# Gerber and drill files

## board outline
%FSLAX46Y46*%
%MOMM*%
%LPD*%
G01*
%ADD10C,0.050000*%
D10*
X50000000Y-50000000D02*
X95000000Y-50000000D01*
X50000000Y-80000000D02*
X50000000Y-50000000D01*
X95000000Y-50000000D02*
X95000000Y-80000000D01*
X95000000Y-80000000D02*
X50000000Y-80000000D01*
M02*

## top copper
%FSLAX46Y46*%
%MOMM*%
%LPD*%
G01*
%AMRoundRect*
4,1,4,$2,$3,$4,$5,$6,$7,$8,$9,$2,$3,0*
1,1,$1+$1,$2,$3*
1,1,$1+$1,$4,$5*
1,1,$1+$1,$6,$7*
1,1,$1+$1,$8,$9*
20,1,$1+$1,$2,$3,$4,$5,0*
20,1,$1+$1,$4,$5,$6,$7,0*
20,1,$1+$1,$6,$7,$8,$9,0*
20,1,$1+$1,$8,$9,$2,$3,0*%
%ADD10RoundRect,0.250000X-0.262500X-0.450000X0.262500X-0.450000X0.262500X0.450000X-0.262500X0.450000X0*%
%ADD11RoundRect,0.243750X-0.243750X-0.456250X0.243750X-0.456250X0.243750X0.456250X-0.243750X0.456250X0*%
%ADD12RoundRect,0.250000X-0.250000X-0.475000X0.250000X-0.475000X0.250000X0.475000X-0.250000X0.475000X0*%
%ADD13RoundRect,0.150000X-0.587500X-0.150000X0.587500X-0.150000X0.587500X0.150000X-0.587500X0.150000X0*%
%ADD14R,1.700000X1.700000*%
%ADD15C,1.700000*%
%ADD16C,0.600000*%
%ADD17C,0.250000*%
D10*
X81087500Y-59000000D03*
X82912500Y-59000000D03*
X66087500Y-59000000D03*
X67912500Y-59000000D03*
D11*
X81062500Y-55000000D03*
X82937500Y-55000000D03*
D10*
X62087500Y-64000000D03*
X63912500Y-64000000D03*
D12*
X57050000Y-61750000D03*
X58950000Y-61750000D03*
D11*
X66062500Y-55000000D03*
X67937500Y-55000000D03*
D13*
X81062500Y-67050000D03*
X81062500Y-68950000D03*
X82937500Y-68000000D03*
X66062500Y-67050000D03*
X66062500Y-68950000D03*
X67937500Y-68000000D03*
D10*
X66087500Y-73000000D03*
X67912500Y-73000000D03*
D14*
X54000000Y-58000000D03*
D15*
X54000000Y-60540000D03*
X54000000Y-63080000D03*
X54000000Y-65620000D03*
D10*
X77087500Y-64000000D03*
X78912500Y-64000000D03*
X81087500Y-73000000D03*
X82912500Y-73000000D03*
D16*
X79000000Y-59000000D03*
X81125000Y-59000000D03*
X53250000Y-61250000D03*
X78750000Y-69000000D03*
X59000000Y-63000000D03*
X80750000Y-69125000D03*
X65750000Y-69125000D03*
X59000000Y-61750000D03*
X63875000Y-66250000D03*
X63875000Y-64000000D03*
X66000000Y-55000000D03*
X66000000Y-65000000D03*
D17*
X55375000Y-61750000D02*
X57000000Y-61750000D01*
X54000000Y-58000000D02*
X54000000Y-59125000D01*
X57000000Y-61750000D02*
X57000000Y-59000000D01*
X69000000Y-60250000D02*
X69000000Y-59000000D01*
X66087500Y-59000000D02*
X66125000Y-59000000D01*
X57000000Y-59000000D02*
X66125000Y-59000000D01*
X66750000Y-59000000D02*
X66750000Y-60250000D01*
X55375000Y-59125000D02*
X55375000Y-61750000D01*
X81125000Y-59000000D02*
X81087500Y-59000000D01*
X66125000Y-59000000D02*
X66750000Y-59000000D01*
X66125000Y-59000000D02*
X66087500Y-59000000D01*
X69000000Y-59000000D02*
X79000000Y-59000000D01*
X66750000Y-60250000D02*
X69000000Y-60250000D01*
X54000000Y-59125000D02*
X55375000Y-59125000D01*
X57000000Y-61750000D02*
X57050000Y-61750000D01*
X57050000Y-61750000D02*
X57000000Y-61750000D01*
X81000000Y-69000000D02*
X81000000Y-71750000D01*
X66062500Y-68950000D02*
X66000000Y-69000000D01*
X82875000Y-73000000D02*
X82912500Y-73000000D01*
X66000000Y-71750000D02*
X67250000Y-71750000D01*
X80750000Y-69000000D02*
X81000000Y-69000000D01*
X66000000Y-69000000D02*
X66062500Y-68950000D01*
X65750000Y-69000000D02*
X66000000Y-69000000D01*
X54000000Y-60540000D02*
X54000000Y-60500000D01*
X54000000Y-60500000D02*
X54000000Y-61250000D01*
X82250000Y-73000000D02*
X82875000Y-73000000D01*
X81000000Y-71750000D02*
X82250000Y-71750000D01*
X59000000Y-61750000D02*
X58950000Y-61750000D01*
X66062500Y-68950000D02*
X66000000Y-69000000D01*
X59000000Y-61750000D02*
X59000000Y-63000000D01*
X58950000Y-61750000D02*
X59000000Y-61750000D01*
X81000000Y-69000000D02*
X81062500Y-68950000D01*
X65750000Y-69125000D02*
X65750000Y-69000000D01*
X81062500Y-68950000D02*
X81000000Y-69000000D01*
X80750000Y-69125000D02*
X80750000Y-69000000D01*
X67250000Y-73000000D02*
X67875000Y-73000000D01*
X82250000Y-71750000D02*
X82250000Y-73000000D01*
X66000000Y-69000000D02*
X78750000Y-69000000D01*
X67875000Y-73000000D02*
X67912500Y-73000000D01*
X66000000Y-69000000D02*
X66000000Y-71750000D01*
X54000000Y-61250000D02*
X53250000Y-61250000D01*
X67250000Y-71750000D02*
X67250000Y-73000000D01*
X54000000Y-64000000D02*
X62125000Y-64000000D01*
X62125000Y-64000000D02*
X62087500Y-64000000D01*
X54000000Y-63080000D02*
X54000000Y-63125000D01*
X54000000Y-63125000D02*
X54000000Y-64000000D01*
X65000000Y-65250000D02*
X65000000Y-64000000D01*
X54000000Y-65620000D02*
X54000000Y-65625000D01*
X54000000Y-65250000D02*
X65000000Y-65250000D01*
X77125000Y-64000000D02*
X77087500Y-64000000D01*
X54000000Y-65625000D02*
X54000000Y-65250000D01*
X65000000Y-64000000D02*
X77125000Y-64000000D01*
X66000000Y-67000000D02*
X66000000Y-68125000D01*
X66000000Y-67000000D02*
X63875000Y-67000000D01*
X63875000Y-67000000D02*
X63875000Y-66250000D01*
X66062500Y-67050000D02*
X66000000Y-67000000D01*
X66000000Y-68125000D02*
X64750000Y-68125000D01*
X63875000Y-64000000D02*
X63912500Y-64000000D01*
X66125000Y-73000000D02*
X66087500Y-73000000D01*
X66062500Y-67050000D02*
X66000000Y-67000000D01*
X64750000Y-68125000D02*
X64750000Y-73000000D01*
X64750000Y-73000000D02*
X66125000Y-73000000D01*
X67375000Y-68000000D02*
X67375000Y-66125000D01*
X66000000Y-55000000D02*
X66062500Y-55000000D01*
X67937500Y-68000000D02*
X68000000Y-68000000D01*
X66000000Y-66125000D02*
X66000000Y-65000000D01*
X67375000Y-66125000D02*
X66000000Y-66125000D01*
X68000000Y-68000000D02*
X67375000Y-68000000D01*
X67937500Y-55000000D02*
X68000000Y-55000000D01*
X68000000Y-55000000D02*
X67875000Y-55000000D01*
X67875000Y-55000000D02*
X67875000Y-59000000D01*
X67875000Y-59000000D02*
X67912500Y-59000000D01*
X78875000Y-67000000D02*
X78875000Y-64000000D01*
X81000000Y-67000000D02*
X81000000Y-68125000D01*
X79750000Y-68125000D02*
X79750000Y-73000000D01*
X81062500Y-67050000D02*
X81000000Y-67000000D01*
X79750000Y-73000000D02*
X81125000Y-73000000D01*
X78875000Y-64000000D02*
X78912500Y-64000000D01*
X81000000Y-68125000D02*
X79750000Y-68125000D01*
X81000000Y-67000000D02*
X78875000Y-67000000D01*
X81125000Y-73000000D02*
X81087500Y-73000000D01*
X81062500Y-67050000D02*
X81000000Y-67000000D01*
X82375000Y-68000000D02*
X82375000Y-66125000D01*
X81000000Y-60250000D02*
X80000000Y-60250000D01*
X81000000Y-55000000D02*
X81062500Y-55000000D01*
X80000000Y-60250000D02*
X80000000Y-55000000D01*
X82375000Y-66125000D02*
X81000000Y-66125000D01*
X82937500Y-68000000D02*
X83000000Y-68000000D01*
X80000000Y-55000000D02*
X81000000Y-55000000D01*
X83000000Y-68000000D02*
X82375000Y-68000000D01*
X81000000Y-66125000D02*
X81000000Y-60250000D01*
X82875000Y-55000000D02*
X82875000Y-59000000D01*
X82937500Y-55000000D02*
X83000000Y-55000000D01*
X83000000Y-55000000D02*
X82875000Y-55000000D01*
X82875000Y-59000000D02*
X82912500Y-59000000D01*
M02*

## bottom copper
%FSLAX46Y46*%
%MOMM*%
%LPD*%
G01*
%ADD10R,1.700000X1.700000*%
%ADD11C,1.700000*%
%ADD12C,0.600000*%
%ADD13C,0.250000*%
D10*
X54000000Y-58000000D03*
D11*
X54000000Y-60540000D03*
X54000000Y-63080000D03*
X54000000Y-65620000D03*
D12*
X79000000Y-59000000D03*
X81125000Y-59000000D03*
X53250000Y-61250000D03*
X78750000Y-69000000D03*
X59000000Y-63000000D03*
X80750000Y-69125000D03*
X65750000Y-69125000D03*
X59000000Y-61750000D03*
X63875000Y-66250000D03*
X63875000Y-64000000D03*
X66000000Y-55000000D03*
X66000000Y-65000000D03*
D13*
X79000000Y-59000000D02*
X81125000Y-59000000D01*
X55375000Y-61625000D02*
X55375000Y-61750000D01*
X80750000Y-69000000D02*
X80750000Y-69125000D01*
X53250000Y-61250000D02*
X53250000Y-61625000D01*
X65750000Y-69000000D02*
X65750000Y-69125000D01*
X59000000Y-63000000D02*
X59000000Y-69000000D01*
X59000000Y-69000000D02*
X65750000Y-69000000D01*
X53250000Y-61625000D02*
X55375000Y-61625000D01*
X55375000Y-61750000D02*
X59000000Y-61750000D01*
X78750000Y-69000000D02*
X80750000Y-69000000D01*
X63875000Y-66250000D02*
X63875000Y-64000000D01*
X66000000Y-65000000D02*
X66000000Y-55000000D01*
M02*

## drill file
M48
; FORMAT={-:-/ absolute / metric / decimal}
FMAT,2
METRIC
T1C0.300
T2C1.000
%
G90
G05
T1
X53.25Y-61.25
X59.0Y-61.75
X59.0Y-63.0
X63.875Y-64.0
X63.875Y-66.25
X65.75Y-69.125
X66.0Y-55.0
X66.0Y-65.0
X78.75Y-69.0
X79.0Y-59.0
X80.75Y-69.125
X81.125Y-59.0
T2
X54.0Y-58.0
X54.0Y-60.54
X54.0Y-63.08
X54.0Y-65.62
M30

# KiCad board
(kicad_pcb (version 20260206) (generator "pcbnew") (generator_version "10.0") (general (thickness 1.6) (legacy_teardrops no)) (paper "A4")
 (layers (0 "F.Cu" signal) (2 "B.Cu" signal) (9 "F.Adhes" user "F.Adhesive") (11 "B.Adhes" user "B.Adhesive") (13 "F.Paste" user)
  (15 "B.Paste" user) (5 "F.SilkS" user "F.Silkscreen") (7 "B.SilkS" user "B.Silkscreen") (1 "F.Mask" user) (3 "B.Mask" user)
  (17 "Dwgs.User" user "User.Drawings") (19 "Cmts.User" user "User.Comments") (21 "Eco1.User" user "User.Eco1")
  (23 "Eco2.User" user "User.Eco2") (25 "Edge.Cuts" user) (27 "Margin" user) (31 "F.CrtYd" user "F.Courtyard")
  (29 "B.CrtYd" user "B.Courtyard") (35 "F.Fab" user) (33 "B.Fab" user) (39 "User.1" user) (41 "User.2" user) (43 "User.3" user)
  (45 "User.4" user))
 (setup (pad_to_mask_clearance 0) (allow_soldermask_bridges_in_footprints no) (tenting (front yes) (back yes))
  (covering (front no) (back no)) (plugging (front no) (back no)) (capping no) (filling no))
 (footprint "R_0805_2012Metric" (layer "F.Cu") (at 82 59)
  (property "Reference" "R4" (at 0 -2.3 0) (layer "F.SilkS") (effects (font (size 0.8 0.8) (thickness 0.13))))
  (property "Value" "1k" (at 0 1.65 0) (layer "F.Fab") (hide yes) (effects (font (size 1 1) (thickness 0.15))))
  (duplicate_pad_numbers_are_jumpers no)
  (pad "1" smd roundrect (at -0.9125 0) (size 1.025 1.4) (layers "F.Cu" "F.Mask" "F.Paste") (roundrect_rratio 0.243902) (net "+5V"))
  (pad "2" smd roundrect (at 0.9125 0) (size 1.025 1.4) (layers "F.Cu" "F.Mask" "F.Paste") (roundrect_rratio 0.243902) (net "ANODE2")))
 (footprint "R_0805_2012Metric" (layer "F.Cu") (at 67 59)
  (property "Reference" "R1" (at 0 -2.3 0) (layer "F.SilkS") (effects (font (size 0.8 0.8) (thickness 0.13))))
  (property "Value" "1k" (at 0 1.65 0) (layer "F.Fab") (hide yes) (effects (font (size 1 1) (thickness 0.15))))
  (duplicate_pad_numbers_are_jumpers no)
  (pad "1" smd roundrect (at -0.9125 0) (size 1.025 1.4) (layers "F.Cu" "F.Mask" "F.Paste") (roundrect_rratio 0.243902) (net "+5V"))
  (pad "2" smd roundrect (at 0.9125 0) (size 1.025 1.4) (layers "F.Cu" "F.Mask" "F.Paste") (roundrect_rratio 0.243902) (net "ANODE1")))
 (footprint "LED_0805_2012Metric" (layer "F.Cu") (at 82 55)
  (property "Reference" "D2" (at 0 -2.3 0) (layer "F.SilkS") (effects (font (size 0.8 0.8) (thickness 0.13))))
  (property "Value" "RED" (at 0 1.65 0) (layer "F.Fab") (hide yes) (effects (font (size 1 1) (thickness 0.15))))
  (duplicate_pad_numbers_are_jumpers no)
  (pad "1" smd roundrect (at -0.9375 0) (size 0.975 1.4) (layers "F.Cu" "F.Mask" "F.Paste") (roundrect_rratio 0.25) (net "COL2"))
  (pad "2" smd roundrect (at 0.9375 0) (size 0.975 1.4) (layers "F.Cu" "F.Mask" "F.Paste") (roundrect_rratio 0.25) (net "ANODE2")))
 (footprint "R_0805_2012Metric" (layer "F.Cu") (at 63 64)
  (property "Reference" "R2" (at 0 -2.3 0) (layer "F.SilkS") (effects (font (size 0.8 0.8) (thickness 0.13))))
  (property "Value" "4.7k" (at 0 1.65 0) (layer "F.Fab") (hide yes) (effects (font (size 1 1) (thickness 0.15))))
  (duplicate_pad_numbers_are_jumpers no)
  (pad "1" smd roundrect (at -0.9125 0) (size 1.025 1.4) (layers "F.Cu" "F.Mask" "F.Paste") (roundrect_rratio 0.243902) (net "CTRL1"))
  (pad "2" smd roundrect (at 0.9125 0) (size 1.025 1.4) (layers "F.Cu" "F.Mask" "F.Paste") (roundrect_rratio 0.243902) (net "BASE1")))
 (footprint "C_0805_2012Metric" (layer "F.Cu") (at 58 61.75)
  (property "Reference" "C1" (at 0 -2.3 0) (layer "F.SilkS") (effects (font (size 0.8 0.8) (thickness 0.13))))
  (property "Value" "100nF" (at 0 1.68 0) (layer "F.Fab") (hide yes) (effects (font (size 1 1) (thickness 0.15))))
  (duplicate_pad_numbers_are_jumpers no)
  (pad "1" smd roundrect (at -0.95 0) (size 1 1.45) (layers "F.Cu" "F.Mask" "F.Paste") (roundrect_rratio 0.25) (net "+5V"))
  (pad "2" smd roundrect (at 0.95 0) (size 1 1.45) (layers "F.Cu" "F.Mask" "F.Paste") (roundrect_rratio 0.25) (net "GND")))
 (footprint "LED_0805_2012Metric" (layer "F.Cu") (at 67 55)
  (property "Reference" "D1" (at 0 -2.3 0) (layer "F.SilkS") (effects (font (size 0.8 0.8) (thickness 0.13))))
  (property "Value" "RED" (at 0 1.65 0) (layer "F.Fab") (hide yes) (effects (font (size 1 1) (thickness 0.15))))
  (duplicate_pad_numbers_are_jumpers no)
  (pad "1" smd roundrect (at -0.9375 0) (size 0.975 1.4) (layers "F.Cu" "F.Mask" "F.Paste") (roundrect_rratio 0.25) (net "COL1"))
  (pad "2" smd roundrect (at 0.9375 0) (size 0.975 1.4) (layers "F.Cu" "F.Mask" "F.Paste") (roundrect_rratio 0.25) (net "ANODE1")))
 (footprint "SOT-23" (layer "F.Cu") (at 82 68)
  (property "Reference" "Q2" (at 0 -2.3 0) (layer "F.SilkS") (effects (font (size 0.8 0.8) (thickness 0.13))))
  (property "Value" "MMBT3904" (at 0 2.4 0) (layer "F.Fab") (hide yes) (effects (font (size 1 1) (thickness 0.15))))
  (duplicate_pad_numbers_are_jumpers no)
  (pad "1" smd roundrect (at -0.9375 -0.95) (size 1.475 0.6) (layers "F.Cu" "F.Mask" "F.Paste") (roundrect_rratio 0.25) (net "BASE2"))
  (pad "2" smd roundrect (at -0.9375 0.95) (size 1.475 0.6) (layers "F.Cu" "F.Mask" "F.Paste") (roundrect_rratio 0.25) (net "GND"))
  (pad "3" smd roundrect (at 0.9375 0) (size 1.475 0.6) (layers "F.Cu" "F.Mask" "F.Paste") (roundrect_rratio 0.25) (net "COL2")))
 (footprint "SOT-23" (layer "F.Cu") (at 67 68)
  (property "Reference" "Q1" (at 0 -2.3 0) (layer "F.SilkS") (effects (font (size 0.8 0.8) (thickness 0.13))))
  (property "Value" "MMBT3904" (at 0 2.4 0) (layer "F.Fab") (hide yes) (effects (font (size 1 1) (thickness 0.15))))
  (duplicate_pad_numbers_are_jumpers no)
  (pad "1" smd roundrect (at -0.9375 -0.95) (size 1.475 0.6) (layers "F.Cu" "F.Mask" "F.Paste") (roundrect_rratio 0.25) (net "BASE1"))
  (pad "2" smd roundrect (at -0.9375 0.95) (size 1.475 0.6) (layers "F.Cu" "F.Mask" "F.Paste") (roundrect_rratio 0.25) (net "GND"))
  (pad "3" smd roundrect (at 0.9375 0) (size 1.475 0.6) (layers "F.Cu" "F.Mask" "F.Paste") (roundrect_rratio 0.25) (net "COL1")))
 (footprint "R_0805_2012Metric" (layer "F.Cu") (at 67 73)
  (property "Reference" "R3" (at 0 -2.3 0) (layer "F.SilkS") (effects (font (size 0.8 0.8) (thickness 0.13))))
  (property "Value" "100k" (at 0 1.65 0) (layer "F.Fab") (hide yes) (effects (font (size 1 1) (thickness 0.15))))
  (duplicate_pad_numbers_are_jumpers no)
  (pad "1" smd roundrect (at -0.9125 0) (size 1.025 1.4) (layers "F.Cu" "F.Mask" "F.Paste") (roundrect_rratio 0.243902) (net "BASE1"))
  (pad "2" smd roundrect (at 0.9125 0) (size 1.025 1.4) (layers "F.Cu" "F.Mask" "F.Paste") (roundrect_rratio 0.243902) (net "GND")))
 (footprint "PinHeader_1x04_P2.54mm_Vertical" (layer "F.Cu") (at 54 58)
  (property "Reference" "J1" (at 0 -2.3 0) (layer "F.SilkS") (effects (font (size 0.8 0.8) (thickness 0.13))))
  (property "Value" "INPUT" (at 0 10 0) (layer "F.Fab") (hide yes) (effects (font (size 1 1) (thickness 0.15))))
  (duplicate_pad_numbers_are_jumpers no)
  (pad "1" thru_hole rect (at 0 0) (size 1.7 1.7) (drill 1) (layers "*.Cu" "*.Mask") (remove_unused_layers no) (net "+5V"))
  (pad "2" thru_hole circle (at 0 2.54) (size 1.7 1.7) (drill 1) (layers "*.Cu" "*.Mask") (remove_unused_layers no) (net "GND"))
  (pad "3" thru_hole circle (at 0 5.08) (size 1.7 1.7) (drill 1) (layers "*.Cu" "*.Mask") (remove_unused_layers no) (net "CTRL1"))
  (pad "4" thru_hole circle (at 0 7.62) (size 1.7 1.7) (drill 1) (layers "*.Cu" "*.Mask") (remove_unused_layers no) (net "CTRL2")))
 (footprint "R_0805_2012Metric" (layer "F.Cu") (at 78 64)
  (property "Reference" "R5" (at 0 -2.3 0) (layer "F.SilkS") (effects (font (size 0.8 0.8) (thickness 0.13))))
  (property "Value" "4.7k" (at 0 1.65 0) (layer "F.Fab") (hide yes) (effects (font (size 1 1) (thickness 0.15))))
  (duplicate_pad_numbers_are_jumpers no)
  (pad "1" smd roundrect (at -0.9125 0) (size 1.025 1.4) (layers "F.Cu" "F.Mask" "F.Paste") (roundrect_rratio 0.243902) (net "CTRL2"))
  (pad "2" smd roundrect (at 0.9125 0) (size 1.025 1.4) (layers "F.Cu" "F.Mask" "F.Paste") (roundrect_rratio 0.243902) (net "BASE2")))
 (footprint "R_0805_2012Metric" (layer "F.Cu") (at 82 73)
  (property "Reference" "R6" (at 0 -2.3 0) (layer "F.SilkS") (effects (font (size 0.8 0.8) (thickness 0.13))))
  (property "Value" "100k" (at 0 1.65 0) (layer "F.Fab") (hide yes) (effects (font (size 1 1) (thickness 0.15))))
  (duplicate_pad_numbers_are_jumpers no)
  (pad "1" smd roundrect (at -0.9125 0) (size 1.025 1.4) (layers "F.Cu" "F.Mask" "F.Paste") (roundrect_rratio 0.243902) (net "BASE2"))
  (pad "2" smd roundrect (at 0.9125 0) (size 1.025 1.4) (layers "F.Cu" "F.Mask" "F.Paste") (roundrect_rratio 0.243902) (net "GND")))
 (gr_line (start 50 50) (end 95 50) (stroke (width 0.05) (type default)) (layer "Edge.Cuts"))
 (gr_line (start 50 80) (end 50 50) (stroke (width 0.05) (type default)) (layer "Edge.Cuts"))
 (gr_line (start 95 50) (end 95 80) (stroke (width 0.05) (type default)) (layer "Edge.Cuts"))
 (gr_line (start 95 80) (end 50 80) (stroke (width 0.05) (type default)) (layer "Edge.Cuts"))
 (segment (start 55.375 61.75) (end 57 61.75) (width 0.25) (layer "F.Cu") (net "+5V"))
 (segment (start 54 58) (end 54 59.125) (width 0.25) (layer "F.Cu") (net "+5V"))
 (segment (start 57 61.75) (end 57 59) (width 0.25) (layer "F.Cu") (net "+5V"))
 (segment (start 69 60.25) (end 69 59) (width 0.25) (layer "F.Cu") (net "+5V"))
 (segment (start 66.0875 59) (end 66.125 59) (width 0.25) (layer "F.Cu") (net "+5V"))
 (segment (start 57 59) (end 66.125 59) (width 0.25) (layer "F.Cu") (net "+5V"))
 (segment (start 66.75 59) (end 66.75 60.25) (width 0.25) (layer "F.Cu") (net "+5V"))
 (segment (start 55.375 59.125) (end 55.375 61.75) (width 0.25) (layer "F.Cu") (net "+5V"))
 (segment (start 81.125 59) (end 81.0875 59) (width 0.25) (layer "F.Cu") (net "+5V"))
 (segment (start 66.125 59) (end 66.75 59) (width 0.25) (layer "F.Cu") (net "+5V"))
 (segment (start 66.125 59) (end 66.0875 59) (width 0.25) (layer "F.Cu") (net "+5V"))
 (segment (start 69 59) (end 79 59) (width 0.25) (layer "F.Cu") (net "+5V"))
 (segment (start 66.75 60.25) (end 69 60.25) (width 0.25) (layer "F.Cu") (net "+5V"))
 (segment (start 54 59.125) (end 55.375 59.125) (width 0.25) (layer "F.Cu") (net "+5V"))
 (segment (start 57 61.75) (end 57.05 61.75) (width 0.25) (layer "F.Cu") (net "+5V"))
 (segment (start 57.05 61.75) (end 57 61.75) (width 0.25) (layer "F.Cu") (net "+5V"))
 (via (at 79 59) (size 0.6) (drill 0.3) (layers "F.Cu" "B.Cu") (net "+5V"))
 (via (at 81.125 59) (size 0.6) (drill 0.3) (layers "F.Cu" "B.Cu") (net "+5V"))
 (segment (start 79 59) (end 81.125 59) (width 0.25) (layer "B.Cu") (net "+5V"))
 (segment (start 81 69) (end 81 71.75) (width 0.25) (layer "F.Cu") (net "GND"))
 (segment (start 66.0625 68.95) (end 66 69) (width 0.25) (layer "F.Cu") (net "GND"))
 (segment (start 82.875 73) (end 82.9125 73) (width 0.25) (layer "F.Cu") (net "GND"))
 (segment (start 66 71.75) (end 67.25 71.75) (width 0.25) (layer "F.Cu") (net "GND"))
 (segment (start 80.75 69) (end 81 69) (width 0.25) (layer "F.Cu") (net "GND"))
 (segment (start 66 69) (end 66.0625 68.95) (width 0.25) (layer "F.Cu") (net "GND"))
 (segment (start 65.75 69) (end 66 69) (width 0.25) (layer "F.Cu") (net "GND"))
 (segment (start 54 60.54) (end 54 60.5) (width 0.25) (layer "F.Cu") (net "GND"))
 (segment (start 54 60.5) (end 54 61.25) (width 0.25) (layer "F.Cu") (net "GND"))
 (segment (start 82.25 73) (end 82.875 73) (width 0.25) (layer "F.Cu") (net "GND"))
 (segment (start 81 71.75) (end 82.25 71.75) (width 0.25) (layer "F.Cu") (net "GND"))
 (segment (start 59 61.75) (end 58.95 61.75) (width 0.25) (layer "F.Cu") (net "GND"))
 (segment (start 66.0625 68.95) (end 66 69) (width 0.25) (layer "F.Cu") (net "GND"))
 (segment (start 59 61.75) (end 59 63) (width 0.25) (layer "F.Cu") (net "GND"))
 (segment (start 58.95 61.75) (end 59 61.75) (width 0.25) (layer "F.Cu") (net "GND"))
 (segment (start 81 69) (end 81.0625 68.95) (width 0.25) (layer "F.Cu") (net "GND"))
 (segment (start 65.75 69.125) (end 65.75 69) (width 0.25) (layer "F.Cu") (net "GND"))
 (segment (start 81.0625 68.95) (end 81 69) (width 0.25) (layer "F.Cu") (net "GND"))
 (segment (start 80.75 69.125) (end 80.75 69) (width 0.25) (layer "F.Cu") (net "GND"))
 (segment (start 67.25 73) (end 67.875 73) (width 0.25) (layer "F.Cu") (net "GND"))
 (segment (start 82.25 71.75) (end 82.25 73) (width 0.25) (layer "F.Cu") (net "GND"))
 (segment (start 66 69) (end 78.75 69) (width 0.25) (layer "F.Cu") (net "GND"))
 (segment (start 67.875 73) (end 67.9125 73) (width 0.25) (layer "F.Cu") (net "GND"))
 (segment (start 66 69) (end 66 71.75) (width 0.25) (layer "F.Cu") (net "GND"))
 (segment (start 54 61.25) (end 53.25 61.25) (width 0.25) (layer "F.Cu") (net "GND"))
 (segment (start 67.25 71.75) (end 67.25 73) (width 0.25) (layer "F.Cu") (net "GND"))
 (via (at 53.25 61.25) (size 0.6) (drill 0.3) (layers "F.Cu" "B.Cu") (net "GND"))
 (via (at 78.75 69) (size 0.6) (drill 0.3) (layers "F.Cu" "B.Cu") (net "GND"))
 (via (at 59 63) (size 0.6) (drill 0.3) (layers "F.Cu" "B.Cu") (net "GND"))
 (via (at 80.75 69.125) (size 0.6) (drill 0.3) (layers "F.Cu" "B.Cu") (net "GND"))
 (via (at 65.75 69.125) (size 0.6) (drill 0.3) (layers "F.Cu" "B.Cu") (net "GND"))
 (via (at 59 61.75) (size 0.6) (drill 0.3) (layers "F.Cu" "B.Cu") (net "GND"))
 (segment (start 55.375 61.625) (end 55.375 61.75) (width 0.25) (layer "B.Cu") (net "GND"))
 (segment (start 80.75 69) (end 80.75 69.125) (width 0.25) (layer "B.Cu") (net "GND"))
 (segment (start 53.25 61.25) (end 53.25 61.625) (width 0.25) (layer "B.Cu") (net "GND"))
 (segment (start 65.75 69) (end 65.75 69.125) (width 0.25) (layer "B.Cu") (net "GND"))
 (segment (start 59 63) (end 59 69) (width 0.25) (layer "B.Cu") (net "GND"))
 (segment (start 59 69) (end 65.75 69) (width 0.25) (layer "B.Cu") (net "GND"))
 (segment (start 53.25 61.625) (end 55.375 61.625) (width 0.25) (layer "B.Cu") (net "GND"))
 (segment (start 55.375 61.75) (end 59 61.75) (width 0.25) (layer "B.Cu") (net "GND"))
 (segment (start 78.75 69) (end 80.75 69) (width 0.25) (layer "B.Cu") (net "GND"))
 (segment (start 54 64) (end 62.125 64) (width 0.25) (layer "F.Cu") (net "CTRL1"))
 (segment (start 62.125 64) (end 62.0875 64) (width 0.25) (layer "F.Cu") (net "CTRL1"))
 (segment (start 54 63.08) (end 54 63.125) (width 0.25) (layer "F.Cu") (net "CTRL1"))
 (segment (start 54 63.125) (end 54 64) (width 0.25) (layer "F.Cu") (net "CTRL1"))
 (segment (start 65 65.25) (end 65 64) (width 0.25) (layer "F.Cu") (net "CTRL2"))
 (segment (start 54 65.62) (end 54 65.625) (width 0.25) (layer "F.Cu") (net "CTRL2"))
 (segment (start 54 65.25) (end 65 65.25) (width 0.25) (layer "F.Cu") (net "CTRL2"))
 (segment (start 77.125 64) (end 77.0875 64) (width 0.25) (layer "F.Cu") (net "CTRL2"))
 (segment (start 54 65.625) (end 54 65.25) (width 0.25) (layer "F.Cu") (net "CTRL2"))
 (segment (start 65 64) (end 77.125 64) (width 0.25) (layer "F.Cu") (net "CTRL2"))
 (segment (start 66 67) (end 66 68.125) (width 0.25) (layer "F.Cu") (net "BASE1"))
 (segment (start 66 67) (end 63.875 67) (width 0.25) (layer "F.Cu") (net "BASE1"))
 (segment (start 63.875 67) (end 63.875 66.25) (width 0.25) (layer "F.Cu") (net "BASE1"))
 (segment (start 66.0625 67.05) (end 66 67) (width 0.25) (layer "F.Cu") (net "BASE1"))
 (segment (start 66 68.125) (end 64.75 68.125) (width 0.25) (layer "F.Cu") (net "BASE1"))
 (segment (start 63.875 64) (end 63.9125 64) (width 0.25) (layer "F.Cu") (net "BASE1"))
 (segment (start 66.125 73) (end 66.0875 73) (width 0.25) (layer "F.Cu") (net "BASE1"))
 (segment (start 66.0625 67.05) (end 66 67) (width 0.25) (layer "F.Cu") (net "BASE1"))
 (segment (start 64.75 68.125) (end 64.75 73) (width 0.25) (layer "F.Cu") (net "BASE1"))
 (segment (start 64.75 73) (end 66.125 73) (width 0.25) (layer "F.Cu") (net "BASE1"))
 (via (at 63.875 66.25) (size 0.6) (drill 0.3) (layers "F.Cu" "B.Cu") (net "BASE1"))
 (via (at 63.875 64) (size 0.6) (drill 0.3) (layers "F.Cu" "B.Cu") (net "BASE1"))
 (segment (start 63.875 66.25) (end 63.875 64) (width 0.25) (layer "B.Cu") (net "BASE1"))
 (segment (start 67.375 68) (end 67.375 66.125) (width 0.25) (layer "F.Cu") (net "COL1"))
 (segment (start 66 55) (end 66.0625 55) (width 0.25) (layer "F.Cu") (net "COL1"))
 (segment (start 67.9375 68) (end 68 68) (width 0.25) (layer "F.Cu") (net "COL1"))
 (segment (start 66 66.125) (end 66 65) (width 0.25) (layer "F.Cu") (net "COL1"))
 (segment (start 67.375 66.125) (end 66 66.125) (width 0.25) (layer "F.Cu") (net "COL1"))
 (segment (start 68 68) (end 67.375 68) (width 0.25) (layer "F.Cu") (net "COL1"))
 (via (at 66 55) (size 0.6) (drill 0.3) (layers "F.Cu" "B.Cu") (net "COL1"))
 (via (at 66 65) (size 0.6) (drill 0.3) (layers "F.Cu" "B.Cu") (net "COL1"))
 (segment (start 66 65) (end 66 55) (width 0.25) (layer "B.Cu") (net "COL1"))
 (segment (start 67.9375 55) (end 68 55) (width 0.25) (layer "F.Cu") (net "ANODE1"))
 (segment (start 68 55) (end 67.875 55) (width 0.25) (layer "F.Cu") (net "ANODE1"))
 (segment (start 67.875 55) (end 67.875 59) (width 0.25) (layer "F.Cu") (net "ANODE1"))
 (segment (start 67.875 59) (end 67.9125 59) (width 0.25) (layer "F.Cu") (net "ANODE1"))
 (segment (start 78.875 67) (end 78.875 64) (width 0.25) (layer "F.Cu") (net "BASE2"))
 (segment (start 81 67) (end 81 68.125) (width 0.25) (layer "F.Cu") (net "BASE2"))
 (segment (start 79.75 68.125) (end 79.75 73) (width 0.25) (layer "F.Cu") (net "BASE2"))
 (segment (start 81.0625 67.05) (end 81 67) (width 0.25) (layer "F.Cu") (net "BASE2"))
 (segment (start 79.75 73) (end 81.125 73) (width 0.25) (layer "F.Cu") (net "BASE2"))
 (segment (start 78.875 64) (end 78.9125 64) (width 0.25) (layer "F.Cu") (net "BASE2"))
 (segment (start 81 68.125) (end 79.75 68.125) (width 0.25) (layer "F.Cu") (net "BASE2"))
 (segment (start 81 67) (end 78.875 67) (width 0.25) (layer "F.Cu") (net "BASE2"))
 (segment (start 81.125 73) (end 81.0875 73) (width 0.25) (layer "F.Cu") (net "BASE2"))
 (segment (start 81.0625 67.05) (end 81 67) (width 0.25) (layer "F.Cu") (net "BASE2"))
 (segment (start 82.375 68) (end 82.375 66.125) (width 0.25) (layer "F.Cu") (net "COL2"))
 (segment (start 81 60.25) (end 80 60.25) (width 0.25) (layer "F.Cu") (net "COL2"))
 (segment (start 81 55) (end 81.0625 55) (width 0.25) (layer "F.Cu") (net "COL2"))
 (segment (start 80 60.25) (end 80 55) (width 0.25) (layer "F.Cu") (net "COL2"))
 (segment (start 82.375 66.125) (end 81 66.125) (width 0.25) (layer "F.Cu") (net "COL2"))
 (segment (start 82.9375 68) (end 83 68) (width 0.25) (layer "F.Cu") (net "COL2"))
 (segment (start 80 55) (end 81 55) (width 0.25) (layer "F.Cu") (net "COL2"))
 (segment (start 83 68) (end 82.375 68) (width 0.25) (layer "F.Cu") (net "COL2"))
 (segment (start 81 66.125) (end 81 60.25) (width 0.25) (layer "F.Cu") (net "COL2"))
 (segment (start 82.875 55) (end 82.875 59) (width 0.25) (layer "F.Cu") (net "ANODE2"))
 (segment (start 82.9375 55) (end 83 55) (width 0.25) (layer "F.Cu") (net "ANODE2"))
 (segment (start 83 55) (end 82.875 55) (width 0.25) (layer "F.Cu") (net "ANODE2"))
 (segment (start 82.875 59) (end 82.9125 59) (width 0.25) (layer "F.Cu") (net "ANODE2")))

